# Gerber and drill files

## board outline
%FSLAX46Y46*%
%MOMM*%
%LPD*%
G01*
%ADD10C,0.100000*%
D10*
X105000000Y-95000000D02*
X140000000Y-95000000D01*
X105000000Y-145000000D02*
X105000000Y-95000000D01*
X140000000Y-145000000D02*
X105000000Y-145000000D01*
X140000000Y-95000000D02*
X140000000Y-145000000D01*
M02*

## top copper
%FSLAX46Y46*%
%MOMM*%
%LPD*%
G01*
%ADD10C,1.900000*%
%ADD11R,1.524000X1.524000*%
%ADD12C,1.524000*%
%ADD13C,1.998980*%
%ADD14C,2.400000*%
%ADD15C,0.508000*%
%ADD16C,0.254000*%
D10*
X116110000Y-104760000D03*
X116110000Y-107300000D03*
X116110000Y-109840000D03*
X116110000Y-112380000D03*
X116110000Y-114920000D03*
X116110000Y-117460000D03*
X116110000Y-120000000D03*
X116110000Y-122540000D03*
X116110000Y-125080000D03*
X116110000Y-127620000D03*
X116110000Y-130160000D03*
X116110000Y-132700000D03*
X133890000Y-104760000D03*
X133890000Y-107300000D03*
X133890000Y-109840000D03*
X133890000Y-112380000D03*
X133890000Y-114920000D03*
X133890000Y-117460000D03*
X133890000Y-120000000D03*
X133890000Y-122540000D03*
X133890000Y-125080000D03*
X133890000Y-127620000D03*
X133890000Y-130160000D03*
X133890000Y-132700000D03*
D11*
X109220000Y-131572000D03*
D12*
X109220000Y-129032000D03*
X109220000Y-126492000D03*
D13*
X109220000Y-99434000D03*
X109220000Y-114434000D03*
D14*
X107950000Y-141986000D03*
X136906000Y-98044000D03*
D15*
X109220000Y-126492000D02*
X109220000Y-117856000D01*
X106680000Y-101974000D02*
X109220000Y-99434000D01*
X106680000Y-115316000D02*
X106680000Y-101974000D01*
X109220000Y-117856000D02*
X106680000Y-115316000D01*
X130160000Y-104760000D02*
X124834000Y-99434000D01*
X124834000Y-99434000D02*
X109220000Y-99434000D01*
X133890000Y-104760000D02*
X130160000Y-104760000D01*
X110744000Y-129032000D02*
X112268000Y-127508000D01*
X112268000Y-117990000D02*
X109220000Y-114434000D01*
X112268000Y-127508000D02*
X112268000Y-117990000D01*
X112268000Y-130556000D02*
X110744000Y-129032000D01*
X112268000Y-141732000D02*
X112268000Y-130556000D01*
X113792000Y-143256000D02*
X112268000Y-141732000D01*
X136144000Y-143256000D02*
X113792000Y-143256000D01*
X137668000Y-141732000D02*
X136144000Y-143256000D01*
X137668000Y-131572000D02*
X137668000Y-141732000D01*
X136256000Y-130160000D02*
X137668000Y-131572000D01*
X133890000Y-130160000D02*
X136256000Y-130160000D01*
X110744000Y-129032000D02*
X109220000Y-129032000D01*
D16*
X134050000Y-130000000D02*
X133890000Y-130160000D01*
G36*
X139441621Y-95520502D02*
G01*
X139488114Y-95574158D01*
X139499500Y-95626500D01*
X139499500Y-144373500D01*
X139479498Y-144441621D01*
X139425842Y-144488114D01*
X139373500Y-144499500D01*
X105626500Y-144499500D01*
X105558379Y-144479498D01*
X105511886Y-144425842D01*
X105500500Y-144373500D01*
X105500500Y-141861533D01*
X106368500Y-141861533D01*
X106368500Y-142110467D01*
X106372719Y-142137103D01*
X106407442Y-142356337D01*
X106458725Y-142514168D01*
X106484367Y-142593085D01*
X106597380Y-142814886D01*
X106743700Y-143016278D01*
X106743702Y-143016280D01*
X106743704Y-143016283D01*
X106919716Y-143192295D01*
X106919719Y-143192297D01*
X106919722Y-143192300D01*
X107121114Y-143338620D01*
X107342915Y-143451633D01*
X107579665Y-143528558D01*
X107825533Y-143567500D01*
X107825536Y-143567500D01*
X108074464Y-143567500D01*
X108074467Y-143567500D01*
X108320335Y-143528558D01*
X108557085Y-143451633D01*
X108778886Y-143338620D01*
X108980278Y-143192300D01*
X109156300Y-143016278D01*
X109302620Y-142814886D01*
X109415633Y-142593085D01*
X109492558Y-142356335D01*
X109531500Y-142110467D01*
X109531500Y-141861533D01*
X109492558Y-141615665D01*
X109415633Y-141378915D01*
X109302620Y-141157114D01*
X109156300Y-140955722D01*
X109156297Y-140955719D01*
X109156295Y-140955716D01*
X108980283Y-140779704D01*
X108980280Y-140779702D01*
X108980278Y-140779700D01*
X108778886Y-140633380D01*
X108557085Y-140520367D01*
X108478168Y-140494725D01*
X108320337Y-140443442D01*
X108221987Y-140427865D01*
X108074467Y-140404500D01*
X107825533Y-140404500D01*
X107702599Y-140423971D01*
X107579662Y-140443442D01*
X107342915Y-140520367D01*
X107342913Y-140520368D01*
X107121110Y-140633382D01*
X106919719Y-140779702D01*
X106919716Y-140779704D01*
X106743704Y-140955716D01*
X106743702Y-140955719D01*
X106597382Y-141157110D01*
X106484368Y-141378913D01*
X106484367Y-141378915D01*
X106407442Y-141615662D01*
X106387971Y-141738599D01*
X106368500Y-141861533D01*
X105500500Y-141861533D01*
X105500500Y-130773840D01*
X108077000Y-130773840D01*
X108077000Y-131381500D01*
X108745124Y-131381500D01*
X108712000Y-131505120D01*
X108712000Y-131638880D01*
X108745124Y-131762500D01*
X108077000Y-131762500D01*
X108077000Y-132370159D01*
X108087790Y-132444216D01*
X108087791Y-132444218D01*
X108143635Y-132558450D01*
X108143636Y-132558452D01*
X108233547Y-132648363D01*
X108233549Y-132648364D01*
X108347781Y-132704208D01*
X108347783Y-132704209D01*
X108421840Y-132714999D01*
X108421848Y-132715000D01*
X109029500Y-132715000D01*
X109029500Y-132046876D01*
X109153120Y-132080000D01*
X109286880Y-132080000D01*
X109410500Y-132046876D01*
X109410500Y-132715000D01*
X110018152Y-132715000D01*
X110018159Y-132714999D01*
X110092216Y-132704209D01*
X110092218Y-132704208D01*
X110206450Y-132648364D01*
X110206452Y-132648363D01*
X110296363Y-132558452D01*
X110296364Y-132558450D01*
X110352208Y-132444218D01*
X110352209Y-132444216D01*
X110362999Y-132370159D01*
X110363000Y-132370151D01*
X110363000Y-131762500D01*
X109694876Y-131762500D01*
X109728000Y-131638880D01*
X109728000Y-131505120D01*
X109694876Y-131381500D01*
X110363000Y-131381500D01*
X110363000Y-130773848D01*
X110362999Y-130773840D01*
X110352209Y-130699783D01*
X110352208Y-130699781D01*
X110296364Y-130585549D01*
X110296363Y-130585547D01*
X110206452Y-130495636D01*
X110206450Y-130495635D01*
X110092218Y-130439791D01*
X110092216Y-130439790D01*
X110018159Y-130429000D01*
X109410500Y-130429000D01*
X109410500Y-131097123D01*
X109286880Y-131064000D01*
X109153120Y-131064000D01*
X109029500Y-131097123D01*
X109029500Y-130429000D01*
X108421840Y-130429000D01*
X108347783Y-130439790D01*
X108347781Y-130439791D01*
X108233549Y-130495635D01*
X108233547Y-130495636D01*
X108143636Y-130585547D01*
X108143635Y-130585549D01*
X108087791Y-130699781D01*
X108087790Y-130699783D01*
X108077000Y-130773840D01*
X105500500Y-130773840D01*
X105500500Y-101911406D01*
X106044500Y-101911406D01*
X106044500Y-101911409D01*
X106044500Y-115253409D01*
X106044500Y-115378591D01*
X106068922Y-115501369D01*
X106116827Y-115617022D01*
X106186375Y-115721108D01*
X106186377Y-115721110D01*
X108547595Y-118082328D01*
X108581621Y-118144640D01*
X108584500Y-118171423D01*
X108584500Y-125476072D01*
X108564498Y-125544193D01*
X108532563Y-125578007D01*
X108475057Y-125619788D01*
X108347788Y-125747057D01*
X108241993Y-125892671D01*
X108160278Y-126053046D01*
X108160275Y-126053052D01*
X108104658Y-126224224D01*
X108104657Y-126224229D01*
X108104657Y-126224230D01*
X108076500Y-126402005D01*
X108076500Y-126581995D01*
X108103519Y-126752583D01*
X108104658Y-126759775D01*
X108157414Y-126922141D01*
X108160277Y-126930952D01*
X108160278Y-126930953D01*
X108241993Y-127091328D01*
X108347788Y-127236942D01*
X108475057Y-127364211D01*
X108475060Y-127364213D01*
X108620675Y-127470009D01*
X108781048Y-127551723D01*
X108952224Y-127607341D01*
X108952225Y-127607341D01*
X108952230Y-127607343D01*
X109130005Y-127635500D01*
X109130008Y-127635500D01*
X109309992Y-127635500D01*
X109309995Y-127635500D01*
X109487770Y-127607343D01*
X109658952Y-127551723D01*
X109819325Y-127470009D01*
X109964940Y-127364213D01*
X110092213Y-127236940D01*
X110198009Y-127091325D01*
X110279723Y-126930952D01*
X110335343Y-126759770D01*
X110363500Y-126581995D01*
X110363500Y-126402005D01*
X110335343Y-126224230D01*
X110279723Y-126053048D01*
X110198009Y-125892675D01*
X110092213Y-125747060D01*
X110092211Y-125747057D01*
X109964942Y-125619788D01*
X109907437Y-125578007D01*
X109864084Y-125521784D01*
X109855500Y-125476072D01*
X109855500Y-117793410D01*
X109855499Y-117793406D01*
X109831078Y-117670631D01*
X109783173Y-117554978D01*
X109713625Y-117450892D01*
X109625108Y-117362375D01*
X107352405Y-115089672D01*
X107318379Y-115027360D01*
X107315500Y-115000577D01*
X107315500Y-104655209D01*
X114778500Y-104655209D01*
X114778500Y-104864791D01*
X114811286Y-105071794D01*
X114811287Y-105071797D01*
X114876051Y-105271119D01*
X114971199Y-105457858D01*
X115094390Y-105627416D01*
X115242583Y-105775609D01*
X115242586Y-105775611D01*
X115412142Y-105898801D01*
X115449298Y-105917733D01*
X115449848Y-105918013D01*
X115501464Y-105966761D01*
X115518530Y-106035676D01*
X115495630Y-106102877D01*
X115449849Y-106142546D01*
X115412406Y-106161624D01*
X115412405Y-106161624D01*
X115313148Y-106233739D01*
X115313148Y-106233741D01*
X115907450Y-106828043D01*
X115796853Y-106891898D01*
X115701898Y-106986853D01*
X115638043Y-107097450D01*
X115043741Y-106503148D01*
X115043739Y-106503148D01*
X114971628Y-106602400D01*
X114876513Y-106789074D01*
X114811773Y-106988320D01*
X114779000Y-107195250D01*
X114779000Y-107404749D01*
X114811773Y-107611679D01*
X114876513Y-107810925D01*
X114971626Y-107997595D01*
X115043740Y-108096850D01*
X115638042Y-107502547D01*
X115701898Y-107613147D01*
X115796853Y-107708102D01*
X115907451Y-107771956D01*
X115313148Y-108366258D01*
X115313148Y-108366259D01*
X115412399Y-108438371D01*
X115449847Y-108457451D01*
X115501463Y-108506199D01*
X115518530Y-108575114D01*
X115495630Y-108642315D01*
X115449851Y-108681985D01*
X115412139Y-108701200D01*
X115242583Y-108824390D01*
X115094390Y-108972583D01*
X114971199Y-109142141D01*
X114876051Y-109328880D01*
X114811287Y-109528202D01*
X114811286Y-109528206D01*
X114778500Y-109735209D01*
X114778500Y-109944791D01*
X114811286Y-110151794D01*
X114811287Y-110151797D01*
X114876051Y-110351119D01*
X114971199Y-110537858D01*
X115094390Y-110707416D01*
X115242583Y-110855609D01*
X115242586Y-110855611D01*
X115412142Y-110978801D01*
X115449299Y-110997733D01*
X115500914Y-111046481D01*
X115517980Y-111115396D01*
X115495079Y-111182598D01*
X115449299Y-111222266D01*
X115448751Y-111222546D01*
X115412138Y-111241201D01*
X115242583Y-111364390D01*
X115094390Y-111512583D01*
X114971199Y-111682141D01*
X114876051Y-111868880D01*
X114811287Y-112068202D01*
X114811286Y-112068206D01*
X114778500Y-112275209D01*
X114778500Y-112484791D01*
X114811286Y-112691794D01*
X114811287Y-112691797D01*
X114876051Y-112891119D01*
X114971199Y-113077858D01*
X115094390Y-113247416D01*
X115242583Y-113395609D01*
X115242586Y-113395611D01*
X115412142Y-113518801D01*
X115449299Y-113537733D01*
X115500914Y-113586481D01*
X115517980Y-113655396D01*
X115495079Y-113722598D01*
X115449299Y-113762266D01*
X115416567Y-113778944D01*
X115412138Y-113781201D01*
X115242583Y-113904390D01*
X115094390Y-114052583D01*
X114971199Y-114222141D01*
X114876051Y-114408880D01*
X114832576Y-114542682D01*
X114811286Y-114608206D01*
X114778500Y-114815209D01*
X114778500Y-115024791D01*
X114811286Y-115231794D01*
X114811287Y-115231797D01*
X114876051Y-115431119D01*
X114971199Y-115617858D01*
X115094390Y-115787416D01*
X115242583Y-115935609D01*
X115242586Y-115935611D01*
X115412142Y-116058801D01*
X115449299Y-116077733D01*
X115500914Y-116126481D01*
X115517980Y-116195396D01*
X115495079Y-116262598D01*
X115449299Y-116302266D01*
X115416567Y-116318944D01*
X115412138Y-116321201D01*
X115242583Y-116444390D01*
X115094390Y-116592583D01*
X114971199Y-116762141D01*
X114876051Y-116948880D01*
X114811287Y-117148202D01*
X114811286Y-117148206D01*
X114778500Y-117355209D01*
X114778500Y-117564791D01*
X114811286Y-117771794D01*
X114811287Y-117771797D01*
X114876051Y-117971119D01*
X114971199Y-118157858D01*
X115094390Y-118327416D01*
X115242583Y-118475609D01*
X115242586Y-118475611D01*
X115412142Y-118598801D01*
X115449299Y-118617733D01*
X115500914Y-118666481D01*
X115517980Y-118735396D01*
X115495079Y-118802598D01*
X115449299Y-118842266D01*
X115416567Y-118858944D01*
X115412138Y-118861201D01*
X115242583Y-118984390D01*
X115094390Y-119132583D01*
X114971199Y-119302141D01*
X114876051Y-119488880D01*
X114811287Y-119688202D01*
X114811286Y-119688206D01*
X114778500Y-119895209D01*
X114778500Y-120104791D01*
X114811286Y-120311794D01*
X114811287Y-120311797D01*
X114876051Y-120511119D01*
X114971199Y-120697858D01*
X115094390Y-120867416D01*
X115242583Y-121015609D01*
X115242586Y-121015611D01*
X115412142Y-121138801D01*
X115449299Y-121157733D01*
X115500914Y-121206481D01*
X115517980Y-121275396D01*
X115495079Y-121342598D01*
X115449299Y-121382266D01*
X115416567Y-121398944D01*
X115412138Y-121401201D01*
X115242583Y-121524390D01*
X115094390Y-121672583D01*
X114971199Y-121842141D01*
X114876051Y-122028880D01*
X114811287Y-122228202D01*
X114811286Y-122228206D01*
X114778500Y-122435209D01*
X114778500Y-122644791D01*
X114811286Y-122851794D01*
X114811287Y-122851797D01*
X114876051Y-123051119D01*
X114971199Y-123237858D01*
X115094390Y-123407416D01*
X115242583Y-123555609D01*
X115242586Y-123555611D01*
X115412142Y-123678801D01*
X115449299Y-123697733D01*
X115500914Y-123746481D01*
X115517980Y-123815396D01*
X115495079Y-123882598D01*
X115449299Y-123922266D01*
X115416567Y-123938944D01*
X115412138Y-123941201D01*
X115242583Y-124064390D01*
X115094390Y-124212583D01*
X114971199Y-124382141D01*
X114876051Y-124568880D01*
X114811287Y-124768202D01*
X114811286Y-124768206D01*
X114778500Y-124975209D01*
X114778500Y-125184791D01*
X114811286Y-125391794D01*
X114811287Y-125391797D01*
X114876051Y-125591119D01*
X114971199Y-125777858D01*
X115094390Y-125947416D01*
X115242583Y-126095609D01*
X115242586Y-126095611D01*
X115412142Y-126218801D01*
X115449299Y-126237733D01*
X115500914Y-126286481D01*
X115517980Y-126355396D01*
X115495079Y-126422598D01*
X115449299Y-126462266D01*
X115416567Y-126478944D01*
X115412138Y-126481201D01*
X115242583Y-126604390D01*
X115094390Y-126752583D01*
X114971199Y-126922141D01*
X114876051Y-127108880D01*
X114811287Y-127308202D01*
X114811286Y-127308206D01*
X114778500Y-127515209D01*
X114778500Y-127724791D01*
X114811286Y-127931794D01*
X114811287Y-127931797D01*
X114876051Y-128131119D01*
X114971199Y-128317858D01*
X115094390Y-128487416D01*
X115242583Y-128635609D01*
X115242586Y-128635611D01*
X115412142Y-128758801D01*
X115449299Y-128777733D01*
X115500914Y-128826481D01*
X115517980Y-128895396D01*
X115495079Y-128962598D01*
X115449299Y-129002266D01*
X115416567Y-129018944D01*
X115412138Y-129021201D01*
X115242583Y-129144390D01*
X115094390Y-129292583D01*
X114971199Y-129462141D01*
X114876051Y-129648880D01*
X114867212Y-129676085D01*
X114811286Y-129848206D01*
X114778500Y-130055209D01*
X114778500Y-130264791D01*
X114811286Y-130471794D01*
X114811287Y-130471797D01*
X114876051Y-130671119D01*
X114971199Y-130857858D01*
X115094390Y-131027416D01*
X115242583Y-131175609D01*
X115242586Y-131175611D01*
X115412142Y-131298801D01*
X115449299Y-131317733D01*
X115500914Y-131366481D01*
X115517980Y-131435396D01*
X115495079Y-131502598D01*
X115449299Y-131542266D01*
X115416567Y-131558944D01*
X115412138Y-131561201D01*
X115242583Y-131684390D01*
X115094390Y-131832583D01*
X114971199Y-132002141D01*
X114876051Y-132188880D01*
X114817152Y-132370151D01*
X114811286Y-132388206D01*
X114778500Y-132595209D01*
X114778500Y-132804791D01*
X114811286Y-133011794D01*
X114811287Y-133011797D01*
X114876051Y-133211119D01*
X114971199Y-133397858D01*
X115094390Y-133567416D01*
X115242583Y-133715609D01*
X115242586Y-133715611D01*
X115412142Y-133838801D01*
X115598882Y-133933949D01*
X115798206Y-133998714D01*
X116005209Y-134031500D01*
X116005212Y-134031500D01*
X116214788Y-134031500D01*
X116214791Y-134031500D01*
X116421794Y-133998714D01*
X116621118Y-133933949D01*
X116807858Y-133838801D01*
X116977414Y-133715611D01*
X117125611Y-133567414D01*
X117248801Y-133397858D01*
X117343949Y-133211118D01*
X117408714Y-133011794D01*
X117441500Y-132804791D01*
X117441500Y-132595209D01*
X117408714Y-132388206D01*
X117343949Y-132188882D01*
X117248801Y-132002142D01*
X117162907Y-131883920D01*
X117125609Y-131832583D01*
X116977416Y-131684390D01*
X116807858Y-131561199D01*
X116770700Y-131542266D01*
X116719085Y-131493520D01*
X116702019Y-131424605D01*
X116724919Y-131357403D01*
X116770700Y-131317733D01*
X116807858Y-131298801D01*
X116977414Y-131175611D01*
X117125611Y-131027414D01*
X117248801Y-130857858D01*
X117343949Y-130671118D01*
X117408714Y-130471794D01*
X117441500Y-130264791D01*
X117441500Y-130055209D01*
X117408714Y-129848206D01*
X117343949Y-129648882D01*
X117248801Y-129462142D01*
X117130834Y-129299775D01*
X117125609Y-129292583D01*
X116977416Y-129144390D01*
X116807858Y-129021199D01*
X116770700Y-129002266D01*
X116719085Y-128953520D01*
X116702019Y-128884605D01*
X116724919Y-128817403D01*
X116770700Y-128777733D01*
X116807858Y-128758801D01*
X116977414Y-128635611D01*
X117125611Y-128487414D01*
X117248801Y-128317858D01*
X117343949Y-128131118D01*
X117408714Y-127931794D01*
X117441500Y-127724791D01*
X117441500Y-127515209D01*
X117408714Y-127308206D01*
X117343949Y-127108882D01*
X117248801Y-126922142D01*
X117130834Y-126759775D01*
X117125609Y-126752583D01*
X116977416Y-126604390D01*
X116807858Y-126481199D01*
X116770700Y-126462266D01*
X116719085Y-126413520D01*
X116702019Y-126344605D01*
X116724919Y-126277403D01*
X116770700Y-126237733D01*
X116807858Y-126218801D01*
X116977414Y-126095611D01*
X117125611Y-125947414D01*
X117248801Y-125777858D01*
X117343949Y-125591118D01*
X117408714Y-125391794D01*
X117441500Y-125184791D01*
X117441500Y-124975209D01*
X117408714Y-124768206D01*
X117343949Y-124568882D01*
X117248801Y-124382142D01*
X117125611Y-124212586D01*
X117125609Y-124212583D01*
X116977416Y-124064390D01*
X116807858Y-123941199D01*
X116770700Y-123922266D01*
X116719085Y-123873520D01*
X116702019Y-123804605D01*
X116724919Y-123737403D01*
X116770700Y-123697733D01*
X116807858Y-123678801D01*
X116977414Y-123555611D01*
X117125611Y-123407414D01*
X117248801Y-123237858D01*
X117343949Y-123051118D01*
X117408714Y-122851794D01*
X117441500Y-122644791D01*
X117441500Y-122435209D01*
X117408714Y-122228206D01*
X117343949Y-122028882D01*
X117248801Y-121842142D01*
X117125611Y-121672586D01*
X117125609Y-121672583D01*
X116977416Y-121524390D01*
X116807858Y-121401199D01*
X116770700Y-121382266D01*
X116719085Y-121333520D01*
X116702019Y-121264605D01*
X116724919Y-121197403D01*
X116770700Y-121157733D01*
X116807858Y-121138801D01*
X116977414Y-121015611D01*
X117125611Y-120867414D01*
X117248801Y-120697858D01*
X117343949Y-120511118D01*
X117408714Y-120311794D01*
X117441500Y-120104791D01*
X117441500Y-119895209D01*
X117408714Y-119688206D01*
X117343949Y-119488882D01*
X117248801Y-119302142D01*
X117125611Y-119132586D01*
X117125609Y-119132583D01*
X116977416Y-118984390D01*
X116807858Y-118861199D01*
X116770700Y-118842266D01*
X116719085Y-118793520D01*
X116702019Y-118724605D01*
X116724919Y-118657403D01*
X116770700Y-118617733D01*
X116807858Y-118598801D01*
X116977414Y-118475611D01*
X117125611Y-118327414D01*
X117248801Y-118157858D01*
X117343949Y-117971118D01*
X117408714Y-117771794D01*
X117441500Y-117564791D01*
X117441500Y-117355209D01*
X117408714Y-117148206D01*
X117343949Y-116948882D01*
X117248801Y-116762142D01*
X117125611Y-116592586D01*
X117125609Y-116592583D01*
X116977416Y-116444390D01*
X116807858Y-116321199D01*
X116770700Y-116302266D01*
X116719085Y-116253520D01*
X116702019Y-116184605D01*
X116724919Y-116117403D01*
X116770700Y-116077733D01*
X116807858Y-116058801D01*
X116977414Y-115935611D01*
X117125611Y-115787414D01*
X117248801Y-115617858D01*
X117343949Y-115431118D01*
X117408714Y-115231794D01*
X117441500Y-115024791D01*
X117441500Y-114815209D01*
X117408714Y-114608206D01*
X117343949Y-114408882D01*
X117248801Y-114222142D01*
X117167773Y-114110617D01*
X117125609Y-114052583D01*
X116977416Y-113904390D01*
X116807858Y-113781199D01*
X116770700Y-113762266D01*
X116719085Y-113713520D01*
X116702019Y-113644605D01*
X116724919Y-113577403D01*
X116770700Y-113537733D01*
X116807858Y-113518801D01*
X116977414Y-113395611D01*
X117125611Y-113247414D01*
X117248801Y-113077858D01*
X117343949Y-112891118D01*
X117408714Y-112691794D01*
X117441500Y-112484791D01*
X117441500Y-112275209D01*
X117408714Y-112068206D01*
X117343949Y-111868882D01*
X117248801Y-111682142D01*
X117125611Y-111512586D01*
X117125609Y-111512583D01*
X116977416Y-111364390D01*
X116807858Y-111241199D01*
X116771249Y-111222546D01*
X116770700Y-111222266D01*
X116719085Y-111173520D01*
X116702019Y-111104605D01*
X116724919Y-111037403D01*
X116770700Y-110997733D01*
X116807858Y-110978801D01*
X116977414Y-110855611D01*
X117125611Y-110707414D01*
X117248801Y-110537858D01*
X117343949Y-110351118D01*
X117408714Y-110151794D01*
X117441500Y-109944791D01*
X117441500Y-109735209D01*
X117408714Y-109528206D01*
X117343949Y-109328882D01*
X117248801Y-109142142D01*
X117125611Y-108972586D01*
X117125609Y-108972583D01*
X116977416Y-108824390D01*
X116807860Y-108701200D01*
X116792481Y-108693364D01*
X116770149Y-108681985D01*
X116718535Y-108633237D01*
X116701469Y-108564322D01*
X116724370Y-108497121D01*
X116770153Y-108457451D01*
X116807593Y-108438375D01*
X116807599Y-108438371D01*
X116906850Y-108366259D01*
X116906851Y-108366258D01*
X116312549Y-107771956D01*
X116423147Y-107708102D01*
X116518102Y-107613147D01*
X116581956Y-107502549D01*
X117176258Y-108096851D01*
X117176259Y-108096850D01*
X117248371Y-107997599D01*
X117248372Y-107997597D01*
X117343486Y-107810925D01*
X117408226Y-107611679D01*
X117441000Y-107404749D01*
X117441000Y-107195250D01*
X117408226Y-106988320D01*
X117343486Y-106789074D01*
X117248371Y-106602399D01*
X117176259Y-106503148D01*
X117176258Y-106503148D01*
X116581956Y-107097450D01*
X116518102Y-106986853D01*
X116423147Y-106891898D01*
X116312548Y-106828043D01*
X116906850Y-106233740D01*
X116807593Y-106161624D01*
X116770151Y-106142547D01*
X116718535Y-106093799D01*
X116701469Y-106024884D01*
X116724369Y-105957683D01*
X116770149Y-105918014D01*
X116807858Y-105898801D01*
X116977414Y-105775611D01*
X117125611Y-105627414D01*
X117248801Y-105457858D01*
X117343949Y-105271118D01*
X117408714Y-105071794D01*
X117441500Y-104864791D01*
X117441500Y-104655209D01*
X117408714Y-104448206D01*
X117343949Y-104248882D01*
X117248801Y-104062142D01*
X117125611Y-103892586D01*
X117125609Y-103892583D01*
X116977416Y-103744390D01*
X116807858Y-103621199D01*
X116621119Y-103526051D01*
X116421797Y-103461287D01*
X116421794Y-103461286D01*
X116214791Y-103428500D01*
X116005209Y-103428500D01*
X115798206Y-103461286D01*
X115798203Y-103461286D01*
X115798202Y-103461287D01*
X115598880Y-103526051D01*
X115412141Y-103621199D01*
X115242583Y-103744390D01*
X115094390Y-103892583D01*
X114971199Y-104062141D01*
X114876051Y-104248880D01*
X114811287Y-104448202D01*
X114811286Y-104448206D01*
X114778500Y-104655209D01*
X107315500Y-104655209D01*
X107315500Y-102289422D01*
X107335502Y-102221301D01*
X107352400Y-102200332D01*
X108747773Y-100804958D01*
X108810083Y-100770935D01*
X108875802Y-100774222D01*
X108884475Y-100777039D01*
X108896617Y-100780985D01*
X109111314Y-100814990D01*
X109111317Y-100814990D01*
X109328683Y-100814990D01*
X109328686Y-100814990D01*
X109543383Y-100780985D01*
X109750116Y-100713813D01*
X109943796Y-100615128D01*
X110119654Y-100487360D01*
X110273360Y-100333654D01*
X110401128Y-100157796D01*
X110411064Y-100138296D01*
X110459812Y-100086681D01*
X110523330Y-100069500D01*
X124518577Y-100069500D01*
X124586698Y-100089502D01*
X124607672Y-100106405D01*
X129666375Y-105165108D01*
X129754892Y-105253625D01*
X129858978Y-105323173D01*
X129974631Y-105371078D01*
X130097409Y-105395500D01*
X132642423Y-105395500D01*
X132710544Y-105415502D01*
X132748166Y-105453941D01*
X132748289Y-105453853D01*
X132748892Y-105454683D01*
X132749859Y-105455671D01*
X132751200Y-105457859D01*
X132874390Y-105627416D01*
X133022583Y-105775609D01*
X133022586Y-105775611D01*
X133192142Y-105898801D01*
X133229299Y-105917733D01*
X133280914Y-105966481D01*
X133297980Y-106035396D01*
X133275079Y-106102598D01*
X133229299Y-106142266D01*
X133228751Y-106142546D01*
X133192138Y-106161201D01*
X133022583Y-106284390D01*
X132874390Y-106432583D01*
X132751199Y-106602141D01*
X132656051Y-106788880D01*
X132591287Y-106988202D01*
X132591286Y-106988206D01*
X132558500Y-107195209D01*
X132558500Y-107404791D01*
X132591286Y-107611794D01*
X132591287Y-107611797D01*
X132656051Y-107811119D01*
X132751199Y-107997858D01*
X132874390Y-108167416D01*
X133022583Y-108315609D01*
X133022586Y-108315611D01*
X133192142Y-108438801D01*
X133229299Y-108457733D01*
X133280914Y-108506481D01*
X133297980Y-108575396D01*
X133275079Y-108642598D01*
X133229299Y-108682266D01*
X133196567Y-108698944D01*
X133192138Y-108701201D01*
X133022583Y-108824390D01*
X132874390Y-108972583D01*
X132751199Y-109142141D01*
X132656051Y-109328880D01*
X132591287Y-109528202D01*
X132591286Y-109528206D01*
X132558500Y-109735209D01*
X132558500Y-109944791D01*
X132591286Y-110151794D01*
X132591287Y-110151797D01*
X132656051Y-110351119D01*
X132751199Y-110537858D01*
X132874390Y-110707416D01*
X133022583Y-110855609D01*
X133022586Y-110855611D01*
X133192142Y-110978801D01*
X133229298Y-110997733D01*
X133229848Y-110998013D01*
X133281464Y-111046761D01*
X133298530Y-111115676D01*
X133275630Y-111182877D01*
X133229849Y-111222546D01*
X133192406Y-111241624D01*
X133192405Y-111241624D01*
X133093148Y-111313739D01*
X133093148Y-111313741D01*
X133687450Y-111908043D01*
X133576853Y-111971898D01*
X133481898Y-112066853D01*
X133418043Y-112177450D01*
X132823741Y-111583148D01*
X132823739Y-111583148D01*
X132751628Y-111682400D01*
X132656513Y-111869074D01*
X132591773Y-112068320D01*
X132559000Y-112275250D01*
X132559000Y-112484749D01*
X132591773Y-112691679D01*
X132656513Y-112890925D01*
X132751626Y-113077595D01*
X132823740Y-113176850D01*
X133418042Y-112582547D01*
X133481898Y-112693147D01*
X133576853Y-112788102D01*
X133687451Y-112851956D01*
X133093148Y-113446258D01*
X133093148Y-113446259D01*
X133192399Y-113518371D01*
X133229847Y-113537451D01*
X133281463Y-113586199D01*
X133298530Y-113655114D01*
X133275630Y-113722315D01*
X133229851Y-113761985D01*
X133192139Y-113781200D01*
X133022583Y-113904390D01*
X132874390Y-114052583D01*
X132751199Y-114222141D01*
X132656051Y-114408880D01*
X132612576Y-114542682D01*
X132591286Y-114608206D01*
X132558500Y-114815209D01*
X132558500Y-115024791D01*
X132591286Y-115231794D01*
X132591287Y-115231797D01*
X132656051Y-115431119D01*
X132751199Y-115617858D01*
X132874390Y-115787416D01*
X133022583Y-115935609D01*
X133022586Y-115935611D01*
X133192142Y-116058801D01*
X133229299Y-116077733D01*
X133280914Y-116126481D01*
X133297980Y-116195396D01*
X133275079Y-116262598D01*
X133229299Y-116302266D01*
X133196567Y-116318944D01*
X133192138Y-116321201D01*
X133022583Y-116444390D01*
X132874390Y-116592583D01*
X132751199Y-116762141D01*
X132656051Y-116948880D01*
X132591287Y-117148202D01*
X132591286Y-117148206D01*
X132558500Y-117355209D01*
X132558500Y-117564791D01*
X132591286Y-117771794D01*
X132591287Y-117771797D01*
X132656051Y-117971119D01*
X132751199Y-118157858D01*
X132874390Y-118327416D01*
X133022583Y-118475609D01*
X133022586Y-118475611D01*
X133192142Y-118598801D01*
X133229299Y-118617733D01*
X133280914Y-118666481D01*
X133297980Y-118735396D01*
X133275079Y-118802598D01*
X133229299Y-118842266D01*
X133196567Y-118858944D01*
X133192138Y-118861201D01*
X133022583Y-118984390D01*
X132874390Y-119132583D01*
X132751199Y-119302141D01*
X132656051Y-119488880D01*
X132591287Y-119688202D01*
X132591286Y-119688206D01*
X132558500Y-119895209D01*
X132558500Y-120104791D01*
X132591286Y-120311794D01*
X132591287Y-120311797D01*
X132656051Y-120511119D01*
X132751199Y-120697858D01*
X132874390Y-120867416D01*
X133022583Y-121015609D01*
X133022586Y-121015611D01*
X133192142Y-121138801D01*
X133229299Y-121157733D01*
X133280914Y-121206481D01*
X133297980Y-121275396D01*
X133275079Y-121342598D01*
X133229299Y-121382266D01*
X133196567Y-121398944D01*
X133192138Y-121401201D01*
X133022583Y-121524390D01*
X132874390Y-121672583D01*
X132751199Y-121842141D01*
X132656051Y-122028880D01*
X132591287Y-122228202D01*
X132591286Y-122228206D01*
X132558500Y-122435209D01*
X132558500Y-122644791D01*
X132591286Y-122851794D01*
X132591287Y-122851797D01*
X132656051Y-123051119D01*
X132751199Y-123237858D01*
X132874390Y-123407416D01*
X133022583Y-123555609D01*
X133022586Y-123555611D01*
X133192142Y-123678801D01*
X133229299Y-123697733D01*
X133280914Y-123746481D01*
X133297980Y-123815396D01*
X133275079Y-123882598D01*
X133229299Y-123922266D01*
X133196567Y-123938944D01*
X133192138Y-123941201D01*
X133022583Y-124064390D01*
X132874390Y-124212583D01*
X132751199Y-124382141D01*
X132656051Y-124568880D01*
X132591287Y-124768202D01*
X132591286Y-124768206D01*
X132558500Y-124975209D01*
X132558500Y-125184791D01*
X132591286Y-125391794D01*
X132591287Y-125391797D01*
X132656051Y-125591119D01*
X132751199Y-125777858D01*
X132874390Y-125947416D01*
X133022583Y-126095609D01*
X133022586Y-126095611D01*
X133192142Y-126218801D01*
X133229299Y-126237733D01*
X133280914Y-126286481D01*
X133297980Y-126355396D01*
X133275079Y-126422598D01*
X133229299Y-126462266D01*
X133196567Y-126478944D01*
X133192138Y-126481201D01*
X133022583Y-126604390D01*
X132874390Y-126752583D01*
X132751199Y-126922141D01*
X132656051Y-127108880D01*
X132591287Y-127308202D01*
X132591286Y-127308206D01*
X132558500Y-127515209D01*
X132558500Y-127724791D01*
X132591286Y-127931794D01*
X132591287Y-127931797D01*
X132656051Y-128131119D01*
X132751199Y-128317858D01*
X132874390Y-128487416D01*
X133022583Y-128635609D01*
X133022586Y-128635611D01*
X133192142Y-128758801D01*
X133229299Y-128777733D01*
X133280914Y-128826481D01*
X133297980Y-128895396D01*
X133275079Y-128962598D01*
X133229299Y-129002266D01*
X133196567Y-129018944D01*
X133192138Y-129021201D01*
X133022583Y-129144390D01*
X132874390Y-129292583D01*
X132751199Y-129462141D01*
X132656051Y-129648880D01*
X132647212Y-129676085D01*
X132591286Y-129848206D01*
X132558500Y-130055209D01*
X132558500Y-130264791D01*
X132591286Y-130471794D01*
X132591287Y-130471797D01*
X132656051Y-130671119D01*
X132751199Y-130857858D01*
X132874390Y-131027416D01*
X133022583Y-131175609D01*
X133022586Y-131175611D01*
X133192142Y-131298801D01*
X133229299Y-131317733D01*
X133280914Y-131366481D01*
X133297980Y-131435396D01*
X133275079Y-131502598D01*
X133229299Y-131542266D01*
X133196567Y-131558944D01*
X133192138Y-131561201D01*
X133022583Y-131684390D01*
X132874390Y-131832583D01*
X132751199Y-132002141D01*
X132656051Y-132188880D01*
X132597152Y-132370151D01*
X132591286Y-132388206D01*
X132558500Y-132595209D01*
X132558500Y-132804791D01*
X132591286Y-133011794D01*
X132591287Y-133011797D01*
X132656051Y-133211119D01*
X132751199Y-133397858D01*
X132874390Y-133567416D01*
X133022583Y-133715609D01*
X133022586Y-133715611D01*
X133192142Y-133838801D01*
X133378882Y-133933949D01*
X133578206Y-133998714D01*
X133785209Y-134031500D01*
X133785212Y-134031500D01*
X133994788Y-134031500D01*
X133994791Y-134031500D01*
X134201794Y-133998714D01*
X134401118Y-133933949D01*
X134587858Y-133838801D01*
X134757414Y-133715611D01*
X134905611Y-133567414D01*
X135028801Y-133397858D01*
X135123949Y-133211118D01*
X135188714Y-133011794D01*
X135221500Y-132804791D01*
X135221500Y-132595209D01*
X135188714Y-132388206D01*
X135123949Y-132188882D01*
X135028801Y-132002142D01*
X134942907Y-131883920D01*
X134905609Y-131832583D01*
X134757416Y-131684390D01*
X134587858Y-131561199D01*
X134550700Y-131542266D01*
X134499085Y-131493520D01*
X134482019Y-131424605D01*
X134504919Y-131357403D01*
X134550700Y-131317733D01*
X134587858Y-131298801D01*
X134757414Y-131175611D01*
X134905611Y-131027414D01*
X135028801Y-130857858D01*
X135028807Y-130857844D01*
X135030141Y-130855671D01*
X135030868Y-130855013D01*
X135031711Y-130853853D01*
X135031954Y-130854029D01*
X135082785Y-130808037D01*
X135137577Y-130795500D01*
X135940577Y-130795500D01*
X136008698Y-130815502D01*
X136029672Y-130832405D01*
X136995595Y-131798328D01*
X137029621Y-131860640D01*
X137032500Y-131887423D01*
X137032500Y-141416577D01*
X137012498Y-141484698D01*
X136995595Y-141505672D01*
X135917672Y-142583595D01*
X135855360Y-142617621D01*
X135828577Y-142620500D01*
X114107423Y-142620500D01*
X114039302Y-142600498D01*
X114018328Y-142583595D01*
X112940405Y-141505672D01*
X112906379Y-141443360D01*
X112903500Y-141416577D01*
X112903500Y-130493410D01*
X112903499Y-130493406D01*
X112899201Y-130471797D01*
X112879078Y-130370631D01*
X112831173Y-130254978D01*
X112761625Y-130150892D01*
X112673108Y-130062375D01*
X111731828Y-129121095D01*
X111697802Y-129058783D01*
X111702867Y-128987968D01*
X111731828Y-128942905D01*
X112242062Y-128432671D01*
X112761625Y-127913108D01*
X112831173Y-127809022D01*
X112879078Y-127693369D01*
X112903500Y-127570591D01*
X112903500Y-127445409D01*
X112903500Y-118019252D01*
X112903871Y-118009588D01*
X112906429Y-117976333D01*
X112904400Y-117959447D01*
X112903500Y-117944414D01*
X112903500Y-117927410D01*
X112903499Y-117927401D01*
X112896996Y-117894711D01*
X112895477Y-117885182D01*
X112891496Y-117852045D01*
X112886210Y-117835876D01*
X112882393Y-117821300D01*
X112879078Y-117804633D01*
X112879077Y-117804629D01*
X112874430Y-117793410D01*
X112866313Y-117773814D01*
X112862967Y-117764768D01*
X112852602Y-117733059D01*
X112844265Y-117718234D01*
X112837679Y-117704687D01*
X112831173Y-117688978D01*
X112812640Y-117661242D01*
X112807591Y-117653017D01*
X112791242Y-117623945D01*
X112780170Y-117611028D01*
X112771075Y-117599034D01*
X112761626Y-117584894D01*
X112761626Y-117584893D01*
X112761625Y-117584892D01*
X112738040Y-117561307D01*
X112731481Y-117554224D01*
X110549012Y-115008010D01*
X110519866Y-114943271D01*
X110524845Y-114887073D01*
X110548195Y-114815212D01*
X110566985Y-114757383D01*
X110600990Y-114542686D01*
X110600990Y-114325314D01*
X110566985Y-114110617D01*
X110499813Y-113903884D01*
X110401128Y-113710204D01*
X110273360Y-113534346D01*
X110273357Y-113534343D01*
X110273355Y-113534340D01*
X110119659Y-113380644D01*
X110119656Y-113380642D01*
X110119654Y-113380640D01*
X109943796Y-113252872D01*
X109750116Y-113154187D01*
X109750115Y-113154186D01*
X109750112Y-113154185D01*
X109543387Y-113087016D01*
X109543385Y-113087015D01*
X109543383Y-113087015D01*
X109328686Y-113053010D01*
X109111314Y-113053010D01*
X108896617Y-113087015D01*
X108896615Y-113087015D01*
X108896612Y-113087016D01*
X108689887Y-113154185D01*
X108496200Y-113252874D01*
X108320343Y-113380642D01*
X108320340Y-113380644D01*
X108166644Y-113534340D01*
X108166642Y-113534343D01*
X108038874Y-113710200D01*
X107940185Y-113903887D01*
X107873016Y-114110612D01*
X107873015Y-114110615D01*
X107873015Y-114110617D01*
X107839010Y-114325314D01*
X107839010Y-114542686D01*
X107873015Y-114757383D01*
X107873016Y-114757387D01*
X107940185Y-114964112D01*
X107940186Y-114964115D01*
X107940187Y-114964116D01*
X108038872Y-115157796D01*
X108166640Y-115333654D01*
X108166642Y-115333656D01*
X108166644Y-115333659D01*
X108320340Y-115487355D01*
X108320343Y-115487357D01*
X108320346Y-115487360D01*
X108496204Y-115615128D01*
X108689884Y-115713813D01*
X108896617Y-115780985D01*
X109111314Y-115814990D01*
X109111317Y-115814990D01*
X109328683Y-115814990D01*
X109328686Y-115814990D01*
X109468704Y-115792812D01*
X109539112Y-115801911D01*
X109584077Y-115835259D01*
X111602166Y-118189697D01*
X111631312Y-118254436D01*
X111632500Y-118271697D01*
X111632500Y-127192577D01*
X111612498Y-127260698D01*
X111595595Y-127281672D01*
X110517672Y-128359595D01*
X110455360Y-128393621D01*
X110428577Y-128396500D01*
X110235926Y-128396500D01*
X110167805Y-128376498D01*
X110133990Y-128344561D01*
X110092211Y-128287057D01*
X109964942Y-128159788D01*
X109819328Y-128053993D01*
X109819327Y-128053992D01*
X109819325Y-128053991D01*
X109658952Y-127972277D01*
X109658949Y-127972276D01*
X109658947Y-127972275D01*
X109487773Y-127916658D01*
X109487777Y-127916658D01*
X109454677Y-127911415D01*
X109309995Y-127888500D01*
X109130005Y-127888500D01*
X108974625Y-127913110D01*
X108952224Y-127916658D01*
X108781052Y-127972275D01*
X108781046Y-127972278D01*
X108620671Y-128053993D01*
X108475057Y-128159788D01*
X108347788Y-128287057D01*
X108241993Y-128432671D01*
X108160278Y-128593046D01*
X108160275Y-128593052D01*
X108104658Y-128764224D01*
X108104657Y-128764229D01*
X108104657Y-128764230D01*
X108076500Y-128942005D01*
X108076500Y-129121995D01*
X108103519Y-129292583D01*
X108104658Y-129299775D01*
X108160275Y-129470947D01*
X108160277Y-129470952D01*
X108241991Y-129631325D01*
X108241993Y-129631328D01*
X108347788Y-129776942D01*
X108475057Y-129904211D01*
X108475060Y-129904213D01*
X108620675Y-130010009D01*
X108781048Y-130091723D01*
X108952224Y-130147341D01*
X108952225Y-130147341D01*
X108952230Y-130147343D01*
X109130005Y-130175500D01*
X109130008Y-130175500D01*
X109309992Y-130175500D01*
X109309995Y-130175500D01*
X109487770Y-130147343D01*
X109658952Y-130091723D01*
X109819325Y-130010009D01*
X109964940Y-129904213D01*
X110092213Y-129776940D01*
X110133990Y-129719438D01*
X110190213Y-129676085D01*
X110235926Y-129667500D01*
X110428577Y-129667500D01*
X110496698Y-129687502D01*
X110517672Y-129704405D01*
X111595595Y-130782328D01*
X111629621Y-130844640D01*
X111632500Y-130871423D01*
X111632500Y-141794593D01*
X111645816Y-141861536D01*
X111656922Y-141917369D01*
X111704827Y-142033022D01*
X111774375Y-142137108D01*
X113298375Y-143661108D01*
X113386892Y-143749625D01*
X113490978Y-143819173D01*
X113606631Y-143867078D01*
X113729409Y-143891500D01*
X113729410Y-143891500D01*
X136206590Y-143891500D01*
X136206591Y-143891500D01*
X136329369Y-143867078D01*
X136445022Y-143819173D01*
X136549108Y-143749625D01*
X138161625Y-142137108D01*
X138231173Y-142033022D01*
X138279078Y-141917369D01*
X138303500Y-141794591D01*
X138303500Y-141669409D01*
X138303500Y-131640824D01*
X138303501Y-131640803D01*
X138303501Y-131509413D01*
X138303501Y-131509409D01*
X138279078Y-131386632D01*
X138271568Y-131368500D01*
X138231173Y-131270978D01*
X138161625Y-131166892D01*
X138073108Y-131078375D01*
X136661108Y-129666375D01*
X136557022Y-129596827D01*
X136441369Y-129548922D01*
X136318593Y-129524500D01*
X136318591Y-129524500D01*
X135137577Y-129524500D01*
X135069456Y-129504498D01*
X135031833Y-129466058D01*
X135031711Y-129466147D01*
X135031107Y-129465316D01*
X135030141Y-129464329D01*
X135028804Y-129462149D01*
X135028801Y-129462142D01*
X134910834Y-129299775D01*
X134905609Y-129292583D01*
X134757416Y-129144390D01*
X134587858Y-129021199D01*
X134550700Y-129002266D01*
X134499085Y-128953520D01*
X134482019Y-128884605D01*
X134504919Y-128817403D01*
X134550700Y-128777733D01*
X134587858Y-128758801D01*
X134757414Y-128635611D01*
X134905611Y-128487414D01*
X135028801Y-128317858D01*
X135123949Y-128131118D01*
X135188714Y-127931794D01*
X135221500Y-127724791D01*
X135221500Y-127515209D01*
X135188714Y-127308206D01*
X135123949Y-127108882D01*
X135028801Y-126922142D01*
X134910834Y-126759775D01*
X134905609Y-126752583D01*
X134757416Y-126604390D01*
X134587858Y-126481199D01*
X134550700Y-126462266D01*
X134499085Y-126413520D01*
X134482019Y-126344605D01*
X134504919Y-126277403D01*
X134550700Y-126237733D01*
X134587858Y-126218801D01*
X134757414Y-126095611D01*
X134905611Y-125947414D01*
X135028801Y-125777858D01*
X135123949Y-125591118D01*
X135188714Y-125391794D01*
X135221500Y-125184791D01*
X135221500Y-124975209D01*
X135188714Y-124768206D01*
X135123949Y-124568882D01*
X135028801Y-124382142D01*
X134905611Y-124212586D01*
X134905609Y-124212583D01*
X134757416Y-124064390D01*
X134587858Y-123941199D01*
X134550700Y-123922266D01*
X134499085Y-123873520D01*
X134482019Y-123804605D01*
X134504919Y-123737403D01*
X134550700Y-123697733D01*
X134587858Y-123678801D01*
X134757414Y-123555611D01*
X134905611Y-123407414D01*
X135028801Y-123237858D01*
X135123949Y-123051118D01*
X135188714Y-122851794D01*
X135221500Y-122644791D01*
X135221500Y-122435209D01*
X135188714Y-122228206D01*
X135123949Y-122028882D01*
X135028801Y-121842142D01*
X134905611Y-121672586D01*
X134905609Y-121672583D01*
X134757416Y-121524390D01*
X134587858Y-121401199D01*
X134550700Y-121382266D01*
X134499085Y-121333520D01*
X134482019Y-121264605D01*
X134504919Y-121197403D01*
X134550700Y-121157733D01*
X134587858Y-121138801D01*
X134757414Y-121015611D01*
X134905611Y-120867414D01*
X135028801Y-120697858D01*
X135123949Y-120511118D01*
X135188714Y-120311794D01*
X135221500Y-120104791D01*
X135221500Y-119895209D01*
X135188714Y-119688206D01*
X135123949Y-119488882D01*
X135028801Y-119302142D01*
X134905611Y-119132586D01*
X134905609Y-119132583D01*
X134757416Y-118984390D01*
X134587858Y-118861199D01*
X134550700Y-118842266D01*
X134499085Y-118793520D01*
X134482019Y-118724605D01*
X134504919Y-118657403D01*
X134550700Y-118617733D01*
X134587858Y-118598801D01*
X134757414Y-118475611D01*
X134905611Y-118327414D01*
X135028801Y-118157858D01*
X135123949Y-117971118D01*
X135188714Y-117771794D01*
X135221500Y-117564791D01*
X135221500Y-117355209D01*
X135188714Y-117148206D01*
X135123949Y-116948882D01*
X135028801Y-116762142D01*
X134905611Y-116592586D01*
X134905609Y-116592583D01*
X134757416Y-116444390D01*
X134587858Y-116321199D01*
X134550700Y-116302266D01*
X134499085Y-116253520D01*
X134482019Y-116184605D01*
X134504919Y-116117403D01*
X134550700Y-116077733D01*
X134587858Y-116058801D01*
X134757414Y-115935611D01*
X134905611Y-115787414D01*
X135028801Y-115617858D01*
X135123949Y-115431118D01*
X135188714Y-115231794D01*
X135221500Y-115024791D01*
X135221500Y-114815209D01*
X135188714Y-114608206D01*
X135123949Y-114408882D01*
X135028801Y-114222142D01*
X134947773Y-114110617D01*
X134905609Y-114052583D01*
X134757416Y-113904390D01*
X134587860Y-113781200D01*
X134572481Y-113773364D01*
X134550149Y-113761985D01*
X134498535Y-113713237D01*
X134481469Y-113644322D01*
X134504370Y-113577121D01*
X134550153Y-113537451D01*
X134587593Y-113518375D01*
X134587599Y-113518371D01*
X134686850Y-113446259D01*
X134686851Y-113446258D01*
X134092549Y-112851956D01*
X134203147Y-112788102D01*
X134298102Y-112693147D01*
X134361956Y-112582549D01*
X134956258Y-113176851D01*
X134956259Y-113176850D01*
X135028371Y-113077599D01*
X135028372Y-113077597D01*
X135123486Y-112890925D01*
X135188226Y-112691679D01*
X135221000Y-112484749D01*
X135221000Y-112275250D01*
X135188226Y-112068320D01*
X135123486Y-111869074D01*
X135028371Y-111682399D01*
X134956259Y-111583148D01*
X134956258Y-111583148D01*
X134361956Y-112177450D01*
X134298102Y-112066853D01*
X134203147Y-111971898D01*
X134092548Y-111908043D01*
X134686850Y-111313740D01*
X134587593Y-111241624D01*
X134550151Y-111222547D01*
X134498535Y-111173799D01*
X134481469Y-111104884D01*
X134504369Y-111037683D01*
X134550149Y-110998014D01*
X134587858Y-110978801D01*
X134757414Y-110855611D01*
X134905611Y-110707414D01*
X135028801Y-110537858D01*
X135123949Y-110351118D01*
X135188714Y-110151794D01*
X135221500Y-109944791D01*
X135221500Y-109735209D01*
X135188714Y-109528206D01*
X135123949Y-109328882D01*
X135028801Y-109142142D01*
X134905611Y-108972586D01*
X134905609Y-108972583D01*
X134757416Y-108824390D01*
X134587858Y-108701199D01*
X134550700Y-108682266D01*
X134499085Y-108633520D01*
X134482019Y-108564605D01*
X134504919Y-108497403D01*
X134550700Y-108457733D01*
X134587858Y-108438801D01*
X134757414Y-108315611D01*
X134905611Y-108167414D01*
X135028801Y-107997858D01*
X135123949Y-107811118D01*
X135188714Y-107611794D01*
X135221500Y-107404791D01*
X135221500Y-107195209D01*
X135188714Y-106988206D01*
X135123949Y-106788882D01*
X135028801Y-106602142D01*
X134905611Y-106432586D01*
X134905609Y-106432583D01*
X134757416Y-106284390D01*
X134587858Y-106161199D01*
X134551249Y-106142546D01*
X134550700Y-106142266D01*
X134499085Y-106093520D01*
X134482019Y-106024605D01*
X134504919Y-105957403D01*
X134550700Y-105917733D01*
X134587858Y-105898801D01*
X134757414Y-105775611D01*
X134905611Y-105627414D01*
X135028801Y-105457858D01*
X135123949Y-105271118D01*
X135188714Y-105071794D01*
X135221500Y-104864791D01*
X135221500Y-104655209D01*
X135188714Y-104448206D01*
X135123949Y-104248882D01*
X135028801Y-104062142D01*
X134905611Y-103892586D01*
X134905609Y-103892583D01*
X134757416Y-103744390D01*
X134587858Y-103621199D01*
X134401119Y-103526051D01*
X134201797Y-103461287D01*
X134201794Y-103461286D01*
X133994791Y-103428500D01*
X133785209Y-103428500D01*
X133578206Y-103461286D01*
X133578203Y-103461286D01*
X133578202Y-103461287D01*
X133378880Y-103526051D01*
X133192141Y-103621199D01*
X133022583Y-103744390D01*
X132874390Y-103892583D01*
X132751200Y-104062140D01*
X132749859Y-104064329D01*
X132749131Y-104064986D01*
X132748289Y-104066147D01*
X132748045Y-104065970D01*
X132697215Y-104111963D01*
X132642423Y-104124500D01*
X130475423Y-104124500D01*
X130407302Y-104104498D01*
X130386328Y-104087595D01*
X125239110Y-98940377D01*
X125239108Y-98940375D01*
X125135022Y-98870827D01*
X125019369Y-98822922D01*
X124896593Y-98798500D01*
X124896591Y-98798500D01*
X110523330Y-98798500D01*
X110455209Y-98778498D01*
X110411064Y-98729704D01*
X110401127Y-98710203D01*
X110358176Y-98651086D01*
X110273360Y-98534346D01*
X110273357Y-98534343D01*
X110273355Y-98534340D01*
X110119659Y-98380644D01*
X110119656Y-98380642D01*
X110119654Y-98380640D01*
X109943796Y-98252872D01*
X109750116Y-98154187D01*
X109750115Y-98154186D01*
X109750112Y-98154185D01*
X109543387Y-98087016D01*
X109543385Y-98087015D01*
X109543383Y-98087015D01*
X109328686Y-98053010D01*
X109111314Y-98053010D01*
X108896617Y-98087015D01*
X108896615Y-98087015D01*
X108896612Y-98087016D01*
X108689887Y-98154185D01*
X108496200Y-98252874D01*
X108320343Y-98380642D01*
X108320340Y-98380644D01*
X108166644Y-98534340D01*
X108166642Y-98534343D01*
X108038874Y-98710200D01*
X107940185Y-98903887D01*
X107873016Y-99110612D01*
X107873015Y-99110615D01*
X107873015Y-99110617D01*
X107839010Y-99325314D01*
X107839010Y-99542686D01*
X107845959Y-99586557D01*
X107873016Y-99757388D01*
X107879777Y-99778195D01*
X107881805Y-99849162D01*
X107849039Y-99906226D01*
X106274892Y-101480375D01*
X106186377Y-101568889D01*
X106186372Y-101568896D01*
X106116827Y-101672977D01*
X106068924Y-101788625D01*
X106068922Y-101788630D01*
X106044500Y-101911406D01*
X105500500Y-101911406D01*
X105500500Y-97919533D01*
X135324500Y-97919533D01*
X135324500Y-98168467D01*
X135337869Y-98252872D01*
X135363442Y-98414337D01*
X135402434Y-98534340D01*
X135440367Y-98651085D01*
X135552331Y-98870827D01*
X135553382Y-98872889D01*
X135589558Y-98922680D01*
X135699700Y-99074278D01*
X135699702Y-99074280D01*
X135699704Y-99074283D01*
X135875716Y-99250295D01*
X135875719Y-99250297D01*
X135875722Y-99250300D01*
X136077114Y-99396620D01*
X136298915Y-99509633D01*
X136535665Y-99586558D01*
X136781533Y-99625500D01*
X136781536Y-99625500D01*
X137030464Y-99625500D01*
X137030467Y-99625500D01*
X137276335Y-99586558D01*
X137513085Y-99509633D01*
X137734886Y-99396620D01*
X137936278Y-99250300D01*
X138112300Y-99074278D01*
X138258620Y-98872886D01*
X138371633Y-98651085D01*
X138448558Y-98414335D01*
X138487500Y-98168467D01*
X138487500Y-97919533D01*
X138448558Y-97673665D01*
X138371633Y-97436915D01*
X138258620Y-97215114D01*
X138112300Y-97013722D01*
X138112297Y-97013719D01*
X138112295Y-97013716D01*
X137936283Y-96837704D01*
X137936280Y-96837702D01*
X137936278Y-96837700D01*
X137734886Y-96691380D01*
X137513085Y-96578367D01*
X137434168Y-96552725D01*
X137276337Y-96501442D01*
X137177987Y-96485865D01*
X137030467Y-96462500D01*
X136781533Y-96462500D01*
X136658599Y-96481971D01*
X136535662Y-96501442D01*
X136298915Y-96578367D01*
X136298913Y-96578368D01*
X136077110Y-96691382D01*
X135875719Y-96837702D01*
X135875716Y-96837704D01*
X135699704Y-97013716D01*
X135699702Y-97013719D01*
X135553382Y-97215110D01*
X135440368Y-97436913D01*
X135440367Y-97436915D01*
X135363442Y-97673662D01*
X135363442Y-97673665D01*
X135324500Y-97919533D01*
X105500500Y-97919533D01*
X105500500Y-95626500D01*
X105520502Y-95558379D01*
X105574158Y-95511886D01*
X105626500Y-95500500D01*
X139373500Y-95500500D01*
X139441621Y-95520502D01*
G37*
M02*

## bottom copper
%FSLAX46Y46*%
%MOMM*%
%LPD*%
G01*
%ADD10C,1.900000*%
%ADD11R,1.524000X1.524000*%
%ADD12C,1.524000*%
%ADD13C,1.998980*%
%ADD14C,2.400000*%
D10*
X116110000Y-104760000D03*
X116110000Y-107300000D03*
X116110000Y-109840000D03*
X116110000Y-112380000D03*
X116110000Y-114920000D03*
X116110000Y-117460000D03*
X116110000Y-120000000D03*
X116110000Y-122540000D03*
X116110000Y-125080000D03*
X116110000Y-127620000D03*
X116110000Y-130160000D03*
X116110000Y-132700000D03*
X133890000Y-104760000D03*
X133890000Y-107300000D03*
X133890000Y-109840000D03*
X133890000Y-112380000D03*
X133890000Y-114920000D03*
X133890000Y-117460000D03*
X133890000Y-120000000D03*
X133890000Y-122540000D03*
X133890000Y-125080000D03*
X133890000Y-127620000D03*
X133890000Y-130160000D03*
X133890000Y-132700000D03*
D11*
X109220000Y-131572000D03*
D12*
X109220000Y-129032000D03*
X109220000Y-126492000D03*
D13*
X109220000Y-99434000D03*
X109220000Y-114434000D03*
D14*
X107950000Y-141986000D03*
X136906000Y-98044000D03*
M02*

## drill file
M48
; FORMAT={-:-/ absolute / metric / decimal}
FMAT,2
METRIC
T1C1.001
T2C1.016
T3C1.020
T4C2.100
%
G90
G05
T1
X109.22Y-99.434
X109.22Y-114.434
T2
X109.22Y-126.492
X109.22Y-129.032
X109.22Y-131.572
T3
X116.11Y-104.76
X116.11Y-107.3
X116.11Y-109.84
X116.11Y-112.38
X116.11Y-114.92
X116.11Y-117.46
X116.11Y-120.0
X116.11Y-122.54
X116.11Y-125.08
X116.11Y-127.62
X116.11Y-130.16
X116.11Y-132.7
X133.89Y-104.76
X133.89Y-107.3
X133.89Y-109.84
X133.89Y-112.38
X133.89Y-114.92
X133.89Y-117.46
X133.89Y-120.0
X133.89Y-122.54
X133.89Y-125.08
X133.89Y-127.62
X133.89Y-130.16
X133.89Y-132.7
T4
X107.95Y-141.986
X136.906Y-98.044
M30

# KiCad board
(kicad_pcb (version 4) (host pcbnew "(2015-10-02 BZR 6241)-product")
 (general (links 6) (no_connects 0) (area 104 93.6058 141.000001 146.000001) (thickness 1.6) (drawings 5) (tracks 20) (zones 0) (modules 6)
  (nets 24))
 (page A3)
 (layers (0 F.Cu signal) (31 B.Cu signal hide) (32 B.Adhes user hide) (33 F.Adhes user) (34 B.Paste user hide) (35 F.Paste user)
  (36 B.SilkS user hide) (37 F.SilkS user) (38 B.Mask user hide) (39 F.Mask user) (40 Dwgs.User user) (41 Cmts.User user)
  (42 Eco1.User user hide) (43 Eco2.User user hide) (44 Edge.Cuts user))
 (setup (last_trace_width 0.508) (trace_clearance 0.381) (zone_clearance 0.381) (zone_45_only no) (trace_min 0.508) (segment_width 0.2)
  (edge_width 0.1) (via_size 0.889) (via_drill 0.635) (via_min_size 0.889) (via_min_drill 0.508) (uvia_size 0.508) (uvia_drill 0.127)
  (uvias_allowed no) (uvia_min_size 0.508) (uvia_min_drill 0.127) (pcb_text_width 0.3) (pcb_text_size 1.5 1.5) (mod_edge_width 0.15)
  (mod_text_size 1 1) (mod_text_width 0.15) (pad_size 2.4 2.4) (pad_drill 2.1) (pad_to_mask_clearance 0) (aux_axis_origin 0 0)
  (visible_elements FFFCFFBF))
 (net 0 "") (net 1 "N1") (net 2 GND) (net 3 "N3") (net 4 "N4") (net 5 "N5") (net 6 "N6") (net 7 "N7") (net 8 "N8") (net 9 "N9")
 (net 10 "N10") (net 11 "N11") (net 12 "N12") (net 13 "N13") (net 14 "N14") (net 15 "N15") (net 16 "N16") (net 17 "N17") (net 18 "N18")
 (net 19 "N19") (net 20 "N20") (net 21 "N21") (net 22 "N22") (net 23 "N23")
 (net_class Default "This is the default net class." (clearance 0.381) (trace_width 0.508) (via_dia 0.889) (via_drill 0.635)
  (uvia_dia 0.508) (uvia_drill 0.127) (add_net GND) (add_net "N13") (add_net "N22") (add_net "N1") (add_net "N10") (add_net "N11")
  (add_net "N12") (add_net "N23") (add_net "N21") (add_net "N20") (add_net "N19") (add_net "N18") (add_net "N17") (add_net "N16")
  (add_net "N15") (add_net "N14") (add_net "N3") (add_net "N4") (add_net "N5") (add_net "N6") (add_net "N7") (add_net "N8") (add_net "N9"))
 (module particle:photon (layer F.Cu) (at 125 120)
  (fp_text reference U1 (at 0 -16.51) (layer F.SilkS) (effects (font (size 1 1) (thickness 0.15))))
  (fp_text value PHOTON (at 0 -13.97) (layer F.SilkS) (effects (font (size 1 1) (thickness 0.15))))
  (pad 1 thru_hole circle (at -8.89 -15.24) (size 1.9 1.9) (drill 1.02) (layers *.Cu *.Mask F.SilkS) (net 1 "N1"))
  (pad 2 thru_hole circle (at -8.89 -12.7) (size 1.9 1.9) (drill 1.02) (layers *.Cu *.Mask F.SilkS) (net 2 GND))
  (pad 3 thru_hole circle (at -8.89 -10.16) (size 1.9 1.9) (drill 1.02) (layers *.Cu *.Mask F.SilkS) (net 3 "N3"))
  (pad 4 thru_hole circle (at -8.89 -7.62) (size 1.9 1.9) (drill 1.02) (layers *.Cu *.Mask F.SilkS) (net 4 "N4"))
  (pad 5 thru_hole circle (at -8.89 -5.08) (size 1.9 1.9) (drill 1.02) (layers *.Cu *.Mask F.SilkS) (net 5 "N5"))
  (pad 6 thru_hole circle (at -8.89 -2.54) (size 1.9 1.9) (drill 1.02) (layers *.Cu *.Mask F.SilkS) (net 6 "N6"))
  (pad 7 thru_hole circle (at -8.89 0) (size 1.9 1.9) (drill 1.02) (layers *.Cu *.Mask F.SilkS) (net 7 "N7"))
  (pad 8 thru_hole circle (at -8.89 2.54) (size 1.9 1.9) (drill 1.02) (layers *.Cu *.Mask F.SilkS) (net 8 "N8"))
  (pad 9 thru_hole circle (at -8.89 5.08) (size 1.9 1.9) (drill 1.02) (layers *.Cu *.Mask F.SilkS) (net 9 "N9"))
  (pad 10 thru_hole circle (at -8.89 7.62) (size 1.9 1.9) (drill 1.02) (layers *.Cu *.Mask F.SilkS) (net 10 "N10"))
  (pad 11 thru_hole circle (at -8.89 10.16) (size 1.9 1.9) (drill 1.02) (layers *.Cu *.Mask F.SilkS) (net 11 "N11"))
  (pad 12 thru_hole circle (at -8.89 12.7) (size 1.9 1.9) (drill 1.02) (layers *.Cu *.Mask F.SilkS) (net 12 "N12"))
  (pad 24 thru_hole circle (at 8.89 -15.24) (size 1.9 1.9) (drill 1.02) (layers *.Cu *.Mask F.SilkS) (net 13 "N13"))
  (pad 23 thru_hole circle (at 8.89 -12.7) (size 1.9 1.9) (drill 1.02) (layers *.Cu *.Mask F.SilkS) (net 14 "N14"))
  (pad 22 thru_hole circle (at 8.89 -10.16) (size 1.9 1.9) (drill 1.02) (layers *.Cu *.Mask F.SilkS) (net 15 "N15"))
  (pad 21 thru_hole circle (at 8.89 -7.62) (size 1.9 1.9) (drill 1.02) (layers *.Cu *.Mask F.SilkS) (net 2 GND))
  (pad 20 thru_hole circle (at 8.89 -5.08) (size 1.9 1.9) (drill 1.02) (layers *.Cu *.Mask F.SilkS) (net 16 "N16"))
  (pad 19 thru_hole circle (at 8.89 -2.54) (size 1.9 1.9) (drill 1.02) (layers *.Cu *.Mask F.SilkS) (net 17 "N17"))
  (pad 18 thru_hole circle (at 8.89 0) (size 1.9 1.9) (drill 1.02) (layers *.Cu *.Mask F.SilkS) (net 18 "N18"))
  (pad 17 thru_hole circle (at 8.89 2.54) (size 1.9 1.9) (drill 1.02) (layers *.Cu *.Mask F.SilkS) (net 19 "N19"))
  (pad 16 thru_hole circle (at 8.89 5.08) (size 1.9 1.9) (drill 1.02) (layers *.Cu *.Mask F.SilkS) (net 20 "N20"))
  (pad 15 thru_hole circle (at 8.89 7.62) (size 1.9 1.9) (drill 1.02) (layers *.Cu *.Mask F.SilkS) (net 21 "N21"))
  (pad 14 thru_hole circle (at 8.89 10.16) (size 1.9 1.9) (drill 1.02) (layers *.Cu *.Mask F.SilkS) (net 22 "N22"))
  (pad 13 thru_hole circle (at 8.89 12.7) (size 1.9 1.9) (drill 1.02) (layers *.Cu *.Mask F.SilkS) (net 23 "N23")))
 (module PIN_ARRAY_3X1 (layer F.Cu) (at 109.22 129.032 90)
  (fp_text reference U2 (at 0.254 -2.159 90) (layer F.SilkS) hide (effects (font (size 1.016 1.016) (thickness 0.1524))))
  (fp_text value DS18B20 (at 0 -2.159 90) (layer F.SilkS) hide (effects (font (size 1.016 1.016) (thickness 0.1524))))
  (pad 1 thru_hole rect (at -2.54 0 90) (size 1.524 1.524) (drill 1.016) (layers *.Cu *.Mask F.SilkS) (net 2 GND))
  (pad 2 thru_hole circle (at 0 0 90) (size 1.524 1.524) (drill 1.016) (layers *.Cu *.Mask F.SilkS) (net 22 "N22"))
  (pad 3 thru_hole circle (at 2.54 0 90) (size 1.524 1.524) (drill 1.016) (layers *.Cu *.Mask F.SilkS) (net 13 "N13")))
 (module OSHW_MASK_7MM (layer F.Cu) (at 125 114)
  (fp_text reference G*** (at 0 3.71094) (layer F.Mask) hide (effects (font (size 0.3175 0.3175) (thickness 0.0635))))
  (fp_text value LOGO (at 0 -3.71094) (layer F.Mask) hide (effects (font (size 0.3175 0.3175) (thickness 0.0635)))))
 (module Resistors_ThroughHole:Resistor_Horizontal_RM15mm (layer F.Cu) (at 109.22 106.934 270)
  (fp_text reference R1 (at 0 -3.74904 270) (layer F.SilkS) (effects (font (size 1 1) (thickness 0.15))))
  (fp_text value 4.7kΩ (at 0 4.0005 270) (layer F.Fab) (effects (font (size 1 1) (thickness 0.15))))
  (pad 1 thru_hole circle (at -7.5 0 270) (size 1.99898 1.99898) (drill 1.00076) (layers *.Cu *.SilkS *.Mask) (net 13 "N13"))
  (pad 2 thru_hole circle (at 7.5 0 270) (size 1.99898 1.99898) (drill 1.00076) (layers *.Cu *.SilkS *.Mask) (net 22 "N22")))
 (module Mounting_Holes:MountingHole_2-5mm (layer F.Cu) (at 107.95 141.986 90)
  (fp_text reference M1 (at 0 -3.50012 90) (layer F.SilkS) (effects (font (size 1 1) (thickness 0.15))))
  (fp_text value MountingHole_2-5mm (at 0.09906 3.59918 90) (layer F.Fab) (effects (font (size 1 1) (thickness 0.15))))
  (pad 1 thru_hole circle (at 0 0 90) (size 2.4 2.4) (drill 2.1) (layers *.Cu) (zone_connect 0)))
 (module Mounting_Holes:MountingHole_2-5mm (layer F.Cu) (at 136.906 98.044)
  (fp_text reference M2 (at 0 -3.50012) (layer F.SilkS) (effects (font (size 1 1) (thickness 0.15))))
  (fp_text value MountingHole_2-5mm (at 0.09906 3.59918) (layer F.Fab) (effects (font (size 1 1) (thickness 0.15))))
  (pad 1 thru_hole circle (at 0 0) (size 2.4 2.4) (drill 2.1) (layers *.Cu)))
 (gr_line (start 105 95) (end 140 95) (angle 90) (layer Edge.Cuts) (width 0.1))
 (gr_line (start 105 145) (end 105 95) (angle 90) (layer Edge.Cuts) (width 0.1))
 (gr_line (start 140 145) (end 105 145) (angle 90) (layer Edge.Cuts) (width 0.1))
 (gr_line (start 140 95) (end 140 145) (angle 90) (layer Edge.Cuts) (width 0.1))
 (segment (start 109.22 126.492) (end 109.22 117.856) (width 0.508) (layer F.Cu) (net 13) (status 10))
 (segment (start 106.68 101.974) (end 109.22 99.434) (width 0.508) (layer F.Cu) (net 13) (status 20))
 (segment (start 106.68 115.316) (end 106.68 101.974) (width 0.508) (layer F.Cu) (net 13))
 (segment (start 109.22 117.856) (end 106.68 115.316) (width 0.508) (layer F.Cu) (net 13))
 (segment (start 130.16 104.76) (end 124.834 99.434) (width 0.508) (layer F.Cu) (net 13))
 (segment (start 124.834 99.434) (end 109.22 99.434) (width 0.508) (layer F.Cu) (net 13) (status 20))
 (segment (start 133.89 104.76) (end 130.16 104.76) (width 0.508) (layer F.Cu) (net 13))
 (segment (start 110.744 129.032) (end 112.268 127.508) (width 0.508) (layer F.Cu) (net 22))
 (segment (start 112.268 117.99) (end 109.22 114.434) (width 0.508) (layer F.Cu) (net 22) (status 20))
 (segment (start 112.268 127.508) (end 112.268 117.99) (width 0.508) (layer F.Cu) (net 22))
 (segment (start 112.268 130.556) (end 110.744 129.032) (width 0.508) (layer F.Cu) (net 22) (status 20))
 (segment (start 112.268 141.732) (end 112.268 130.556) (width 0.508) (layer F.Cu) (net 22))
 (segment (start 113.792 143.256) (end 112.268 141.732) (width 0.508) (layer F.Cu) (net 22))
 (segment (start 136.144 143.256) (end 113.792 143.256) (width 0.508) (layer F.Cu) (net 22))
 (segment (start 137.668 141.732) (end 136.144 143.256) (width 0.508) (layer F.Cu) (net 22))
 (segment (start 137.668 131.572) (end 137.668 141.732) (width 0.508) (layer F.Cu) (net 22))
 (segment (start 136.256 130.16) (end 137.668 131.572) (width 0.508) (layer F.Cu) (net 22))
 (segment (start 133.89 130.16) (end 136.256 130.16) (width 0.508) (layer F.Cu) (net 22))
 (segment (start 110.744 129.032) (end 109.22 129.032) (width 0.508) (layer F.Cu) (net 22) (status 20))
 (segment (start 134.05 130) (end 133.89 130.16) (width 0.254) (layer F.Cu) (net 22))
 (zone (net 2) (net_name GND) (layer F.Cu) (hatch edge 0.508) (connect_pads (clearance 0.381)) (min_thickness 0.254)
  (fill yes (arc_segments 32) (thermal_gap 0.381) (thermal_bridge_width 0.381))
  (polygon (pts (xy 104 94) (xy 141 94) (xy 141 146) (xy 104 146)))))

